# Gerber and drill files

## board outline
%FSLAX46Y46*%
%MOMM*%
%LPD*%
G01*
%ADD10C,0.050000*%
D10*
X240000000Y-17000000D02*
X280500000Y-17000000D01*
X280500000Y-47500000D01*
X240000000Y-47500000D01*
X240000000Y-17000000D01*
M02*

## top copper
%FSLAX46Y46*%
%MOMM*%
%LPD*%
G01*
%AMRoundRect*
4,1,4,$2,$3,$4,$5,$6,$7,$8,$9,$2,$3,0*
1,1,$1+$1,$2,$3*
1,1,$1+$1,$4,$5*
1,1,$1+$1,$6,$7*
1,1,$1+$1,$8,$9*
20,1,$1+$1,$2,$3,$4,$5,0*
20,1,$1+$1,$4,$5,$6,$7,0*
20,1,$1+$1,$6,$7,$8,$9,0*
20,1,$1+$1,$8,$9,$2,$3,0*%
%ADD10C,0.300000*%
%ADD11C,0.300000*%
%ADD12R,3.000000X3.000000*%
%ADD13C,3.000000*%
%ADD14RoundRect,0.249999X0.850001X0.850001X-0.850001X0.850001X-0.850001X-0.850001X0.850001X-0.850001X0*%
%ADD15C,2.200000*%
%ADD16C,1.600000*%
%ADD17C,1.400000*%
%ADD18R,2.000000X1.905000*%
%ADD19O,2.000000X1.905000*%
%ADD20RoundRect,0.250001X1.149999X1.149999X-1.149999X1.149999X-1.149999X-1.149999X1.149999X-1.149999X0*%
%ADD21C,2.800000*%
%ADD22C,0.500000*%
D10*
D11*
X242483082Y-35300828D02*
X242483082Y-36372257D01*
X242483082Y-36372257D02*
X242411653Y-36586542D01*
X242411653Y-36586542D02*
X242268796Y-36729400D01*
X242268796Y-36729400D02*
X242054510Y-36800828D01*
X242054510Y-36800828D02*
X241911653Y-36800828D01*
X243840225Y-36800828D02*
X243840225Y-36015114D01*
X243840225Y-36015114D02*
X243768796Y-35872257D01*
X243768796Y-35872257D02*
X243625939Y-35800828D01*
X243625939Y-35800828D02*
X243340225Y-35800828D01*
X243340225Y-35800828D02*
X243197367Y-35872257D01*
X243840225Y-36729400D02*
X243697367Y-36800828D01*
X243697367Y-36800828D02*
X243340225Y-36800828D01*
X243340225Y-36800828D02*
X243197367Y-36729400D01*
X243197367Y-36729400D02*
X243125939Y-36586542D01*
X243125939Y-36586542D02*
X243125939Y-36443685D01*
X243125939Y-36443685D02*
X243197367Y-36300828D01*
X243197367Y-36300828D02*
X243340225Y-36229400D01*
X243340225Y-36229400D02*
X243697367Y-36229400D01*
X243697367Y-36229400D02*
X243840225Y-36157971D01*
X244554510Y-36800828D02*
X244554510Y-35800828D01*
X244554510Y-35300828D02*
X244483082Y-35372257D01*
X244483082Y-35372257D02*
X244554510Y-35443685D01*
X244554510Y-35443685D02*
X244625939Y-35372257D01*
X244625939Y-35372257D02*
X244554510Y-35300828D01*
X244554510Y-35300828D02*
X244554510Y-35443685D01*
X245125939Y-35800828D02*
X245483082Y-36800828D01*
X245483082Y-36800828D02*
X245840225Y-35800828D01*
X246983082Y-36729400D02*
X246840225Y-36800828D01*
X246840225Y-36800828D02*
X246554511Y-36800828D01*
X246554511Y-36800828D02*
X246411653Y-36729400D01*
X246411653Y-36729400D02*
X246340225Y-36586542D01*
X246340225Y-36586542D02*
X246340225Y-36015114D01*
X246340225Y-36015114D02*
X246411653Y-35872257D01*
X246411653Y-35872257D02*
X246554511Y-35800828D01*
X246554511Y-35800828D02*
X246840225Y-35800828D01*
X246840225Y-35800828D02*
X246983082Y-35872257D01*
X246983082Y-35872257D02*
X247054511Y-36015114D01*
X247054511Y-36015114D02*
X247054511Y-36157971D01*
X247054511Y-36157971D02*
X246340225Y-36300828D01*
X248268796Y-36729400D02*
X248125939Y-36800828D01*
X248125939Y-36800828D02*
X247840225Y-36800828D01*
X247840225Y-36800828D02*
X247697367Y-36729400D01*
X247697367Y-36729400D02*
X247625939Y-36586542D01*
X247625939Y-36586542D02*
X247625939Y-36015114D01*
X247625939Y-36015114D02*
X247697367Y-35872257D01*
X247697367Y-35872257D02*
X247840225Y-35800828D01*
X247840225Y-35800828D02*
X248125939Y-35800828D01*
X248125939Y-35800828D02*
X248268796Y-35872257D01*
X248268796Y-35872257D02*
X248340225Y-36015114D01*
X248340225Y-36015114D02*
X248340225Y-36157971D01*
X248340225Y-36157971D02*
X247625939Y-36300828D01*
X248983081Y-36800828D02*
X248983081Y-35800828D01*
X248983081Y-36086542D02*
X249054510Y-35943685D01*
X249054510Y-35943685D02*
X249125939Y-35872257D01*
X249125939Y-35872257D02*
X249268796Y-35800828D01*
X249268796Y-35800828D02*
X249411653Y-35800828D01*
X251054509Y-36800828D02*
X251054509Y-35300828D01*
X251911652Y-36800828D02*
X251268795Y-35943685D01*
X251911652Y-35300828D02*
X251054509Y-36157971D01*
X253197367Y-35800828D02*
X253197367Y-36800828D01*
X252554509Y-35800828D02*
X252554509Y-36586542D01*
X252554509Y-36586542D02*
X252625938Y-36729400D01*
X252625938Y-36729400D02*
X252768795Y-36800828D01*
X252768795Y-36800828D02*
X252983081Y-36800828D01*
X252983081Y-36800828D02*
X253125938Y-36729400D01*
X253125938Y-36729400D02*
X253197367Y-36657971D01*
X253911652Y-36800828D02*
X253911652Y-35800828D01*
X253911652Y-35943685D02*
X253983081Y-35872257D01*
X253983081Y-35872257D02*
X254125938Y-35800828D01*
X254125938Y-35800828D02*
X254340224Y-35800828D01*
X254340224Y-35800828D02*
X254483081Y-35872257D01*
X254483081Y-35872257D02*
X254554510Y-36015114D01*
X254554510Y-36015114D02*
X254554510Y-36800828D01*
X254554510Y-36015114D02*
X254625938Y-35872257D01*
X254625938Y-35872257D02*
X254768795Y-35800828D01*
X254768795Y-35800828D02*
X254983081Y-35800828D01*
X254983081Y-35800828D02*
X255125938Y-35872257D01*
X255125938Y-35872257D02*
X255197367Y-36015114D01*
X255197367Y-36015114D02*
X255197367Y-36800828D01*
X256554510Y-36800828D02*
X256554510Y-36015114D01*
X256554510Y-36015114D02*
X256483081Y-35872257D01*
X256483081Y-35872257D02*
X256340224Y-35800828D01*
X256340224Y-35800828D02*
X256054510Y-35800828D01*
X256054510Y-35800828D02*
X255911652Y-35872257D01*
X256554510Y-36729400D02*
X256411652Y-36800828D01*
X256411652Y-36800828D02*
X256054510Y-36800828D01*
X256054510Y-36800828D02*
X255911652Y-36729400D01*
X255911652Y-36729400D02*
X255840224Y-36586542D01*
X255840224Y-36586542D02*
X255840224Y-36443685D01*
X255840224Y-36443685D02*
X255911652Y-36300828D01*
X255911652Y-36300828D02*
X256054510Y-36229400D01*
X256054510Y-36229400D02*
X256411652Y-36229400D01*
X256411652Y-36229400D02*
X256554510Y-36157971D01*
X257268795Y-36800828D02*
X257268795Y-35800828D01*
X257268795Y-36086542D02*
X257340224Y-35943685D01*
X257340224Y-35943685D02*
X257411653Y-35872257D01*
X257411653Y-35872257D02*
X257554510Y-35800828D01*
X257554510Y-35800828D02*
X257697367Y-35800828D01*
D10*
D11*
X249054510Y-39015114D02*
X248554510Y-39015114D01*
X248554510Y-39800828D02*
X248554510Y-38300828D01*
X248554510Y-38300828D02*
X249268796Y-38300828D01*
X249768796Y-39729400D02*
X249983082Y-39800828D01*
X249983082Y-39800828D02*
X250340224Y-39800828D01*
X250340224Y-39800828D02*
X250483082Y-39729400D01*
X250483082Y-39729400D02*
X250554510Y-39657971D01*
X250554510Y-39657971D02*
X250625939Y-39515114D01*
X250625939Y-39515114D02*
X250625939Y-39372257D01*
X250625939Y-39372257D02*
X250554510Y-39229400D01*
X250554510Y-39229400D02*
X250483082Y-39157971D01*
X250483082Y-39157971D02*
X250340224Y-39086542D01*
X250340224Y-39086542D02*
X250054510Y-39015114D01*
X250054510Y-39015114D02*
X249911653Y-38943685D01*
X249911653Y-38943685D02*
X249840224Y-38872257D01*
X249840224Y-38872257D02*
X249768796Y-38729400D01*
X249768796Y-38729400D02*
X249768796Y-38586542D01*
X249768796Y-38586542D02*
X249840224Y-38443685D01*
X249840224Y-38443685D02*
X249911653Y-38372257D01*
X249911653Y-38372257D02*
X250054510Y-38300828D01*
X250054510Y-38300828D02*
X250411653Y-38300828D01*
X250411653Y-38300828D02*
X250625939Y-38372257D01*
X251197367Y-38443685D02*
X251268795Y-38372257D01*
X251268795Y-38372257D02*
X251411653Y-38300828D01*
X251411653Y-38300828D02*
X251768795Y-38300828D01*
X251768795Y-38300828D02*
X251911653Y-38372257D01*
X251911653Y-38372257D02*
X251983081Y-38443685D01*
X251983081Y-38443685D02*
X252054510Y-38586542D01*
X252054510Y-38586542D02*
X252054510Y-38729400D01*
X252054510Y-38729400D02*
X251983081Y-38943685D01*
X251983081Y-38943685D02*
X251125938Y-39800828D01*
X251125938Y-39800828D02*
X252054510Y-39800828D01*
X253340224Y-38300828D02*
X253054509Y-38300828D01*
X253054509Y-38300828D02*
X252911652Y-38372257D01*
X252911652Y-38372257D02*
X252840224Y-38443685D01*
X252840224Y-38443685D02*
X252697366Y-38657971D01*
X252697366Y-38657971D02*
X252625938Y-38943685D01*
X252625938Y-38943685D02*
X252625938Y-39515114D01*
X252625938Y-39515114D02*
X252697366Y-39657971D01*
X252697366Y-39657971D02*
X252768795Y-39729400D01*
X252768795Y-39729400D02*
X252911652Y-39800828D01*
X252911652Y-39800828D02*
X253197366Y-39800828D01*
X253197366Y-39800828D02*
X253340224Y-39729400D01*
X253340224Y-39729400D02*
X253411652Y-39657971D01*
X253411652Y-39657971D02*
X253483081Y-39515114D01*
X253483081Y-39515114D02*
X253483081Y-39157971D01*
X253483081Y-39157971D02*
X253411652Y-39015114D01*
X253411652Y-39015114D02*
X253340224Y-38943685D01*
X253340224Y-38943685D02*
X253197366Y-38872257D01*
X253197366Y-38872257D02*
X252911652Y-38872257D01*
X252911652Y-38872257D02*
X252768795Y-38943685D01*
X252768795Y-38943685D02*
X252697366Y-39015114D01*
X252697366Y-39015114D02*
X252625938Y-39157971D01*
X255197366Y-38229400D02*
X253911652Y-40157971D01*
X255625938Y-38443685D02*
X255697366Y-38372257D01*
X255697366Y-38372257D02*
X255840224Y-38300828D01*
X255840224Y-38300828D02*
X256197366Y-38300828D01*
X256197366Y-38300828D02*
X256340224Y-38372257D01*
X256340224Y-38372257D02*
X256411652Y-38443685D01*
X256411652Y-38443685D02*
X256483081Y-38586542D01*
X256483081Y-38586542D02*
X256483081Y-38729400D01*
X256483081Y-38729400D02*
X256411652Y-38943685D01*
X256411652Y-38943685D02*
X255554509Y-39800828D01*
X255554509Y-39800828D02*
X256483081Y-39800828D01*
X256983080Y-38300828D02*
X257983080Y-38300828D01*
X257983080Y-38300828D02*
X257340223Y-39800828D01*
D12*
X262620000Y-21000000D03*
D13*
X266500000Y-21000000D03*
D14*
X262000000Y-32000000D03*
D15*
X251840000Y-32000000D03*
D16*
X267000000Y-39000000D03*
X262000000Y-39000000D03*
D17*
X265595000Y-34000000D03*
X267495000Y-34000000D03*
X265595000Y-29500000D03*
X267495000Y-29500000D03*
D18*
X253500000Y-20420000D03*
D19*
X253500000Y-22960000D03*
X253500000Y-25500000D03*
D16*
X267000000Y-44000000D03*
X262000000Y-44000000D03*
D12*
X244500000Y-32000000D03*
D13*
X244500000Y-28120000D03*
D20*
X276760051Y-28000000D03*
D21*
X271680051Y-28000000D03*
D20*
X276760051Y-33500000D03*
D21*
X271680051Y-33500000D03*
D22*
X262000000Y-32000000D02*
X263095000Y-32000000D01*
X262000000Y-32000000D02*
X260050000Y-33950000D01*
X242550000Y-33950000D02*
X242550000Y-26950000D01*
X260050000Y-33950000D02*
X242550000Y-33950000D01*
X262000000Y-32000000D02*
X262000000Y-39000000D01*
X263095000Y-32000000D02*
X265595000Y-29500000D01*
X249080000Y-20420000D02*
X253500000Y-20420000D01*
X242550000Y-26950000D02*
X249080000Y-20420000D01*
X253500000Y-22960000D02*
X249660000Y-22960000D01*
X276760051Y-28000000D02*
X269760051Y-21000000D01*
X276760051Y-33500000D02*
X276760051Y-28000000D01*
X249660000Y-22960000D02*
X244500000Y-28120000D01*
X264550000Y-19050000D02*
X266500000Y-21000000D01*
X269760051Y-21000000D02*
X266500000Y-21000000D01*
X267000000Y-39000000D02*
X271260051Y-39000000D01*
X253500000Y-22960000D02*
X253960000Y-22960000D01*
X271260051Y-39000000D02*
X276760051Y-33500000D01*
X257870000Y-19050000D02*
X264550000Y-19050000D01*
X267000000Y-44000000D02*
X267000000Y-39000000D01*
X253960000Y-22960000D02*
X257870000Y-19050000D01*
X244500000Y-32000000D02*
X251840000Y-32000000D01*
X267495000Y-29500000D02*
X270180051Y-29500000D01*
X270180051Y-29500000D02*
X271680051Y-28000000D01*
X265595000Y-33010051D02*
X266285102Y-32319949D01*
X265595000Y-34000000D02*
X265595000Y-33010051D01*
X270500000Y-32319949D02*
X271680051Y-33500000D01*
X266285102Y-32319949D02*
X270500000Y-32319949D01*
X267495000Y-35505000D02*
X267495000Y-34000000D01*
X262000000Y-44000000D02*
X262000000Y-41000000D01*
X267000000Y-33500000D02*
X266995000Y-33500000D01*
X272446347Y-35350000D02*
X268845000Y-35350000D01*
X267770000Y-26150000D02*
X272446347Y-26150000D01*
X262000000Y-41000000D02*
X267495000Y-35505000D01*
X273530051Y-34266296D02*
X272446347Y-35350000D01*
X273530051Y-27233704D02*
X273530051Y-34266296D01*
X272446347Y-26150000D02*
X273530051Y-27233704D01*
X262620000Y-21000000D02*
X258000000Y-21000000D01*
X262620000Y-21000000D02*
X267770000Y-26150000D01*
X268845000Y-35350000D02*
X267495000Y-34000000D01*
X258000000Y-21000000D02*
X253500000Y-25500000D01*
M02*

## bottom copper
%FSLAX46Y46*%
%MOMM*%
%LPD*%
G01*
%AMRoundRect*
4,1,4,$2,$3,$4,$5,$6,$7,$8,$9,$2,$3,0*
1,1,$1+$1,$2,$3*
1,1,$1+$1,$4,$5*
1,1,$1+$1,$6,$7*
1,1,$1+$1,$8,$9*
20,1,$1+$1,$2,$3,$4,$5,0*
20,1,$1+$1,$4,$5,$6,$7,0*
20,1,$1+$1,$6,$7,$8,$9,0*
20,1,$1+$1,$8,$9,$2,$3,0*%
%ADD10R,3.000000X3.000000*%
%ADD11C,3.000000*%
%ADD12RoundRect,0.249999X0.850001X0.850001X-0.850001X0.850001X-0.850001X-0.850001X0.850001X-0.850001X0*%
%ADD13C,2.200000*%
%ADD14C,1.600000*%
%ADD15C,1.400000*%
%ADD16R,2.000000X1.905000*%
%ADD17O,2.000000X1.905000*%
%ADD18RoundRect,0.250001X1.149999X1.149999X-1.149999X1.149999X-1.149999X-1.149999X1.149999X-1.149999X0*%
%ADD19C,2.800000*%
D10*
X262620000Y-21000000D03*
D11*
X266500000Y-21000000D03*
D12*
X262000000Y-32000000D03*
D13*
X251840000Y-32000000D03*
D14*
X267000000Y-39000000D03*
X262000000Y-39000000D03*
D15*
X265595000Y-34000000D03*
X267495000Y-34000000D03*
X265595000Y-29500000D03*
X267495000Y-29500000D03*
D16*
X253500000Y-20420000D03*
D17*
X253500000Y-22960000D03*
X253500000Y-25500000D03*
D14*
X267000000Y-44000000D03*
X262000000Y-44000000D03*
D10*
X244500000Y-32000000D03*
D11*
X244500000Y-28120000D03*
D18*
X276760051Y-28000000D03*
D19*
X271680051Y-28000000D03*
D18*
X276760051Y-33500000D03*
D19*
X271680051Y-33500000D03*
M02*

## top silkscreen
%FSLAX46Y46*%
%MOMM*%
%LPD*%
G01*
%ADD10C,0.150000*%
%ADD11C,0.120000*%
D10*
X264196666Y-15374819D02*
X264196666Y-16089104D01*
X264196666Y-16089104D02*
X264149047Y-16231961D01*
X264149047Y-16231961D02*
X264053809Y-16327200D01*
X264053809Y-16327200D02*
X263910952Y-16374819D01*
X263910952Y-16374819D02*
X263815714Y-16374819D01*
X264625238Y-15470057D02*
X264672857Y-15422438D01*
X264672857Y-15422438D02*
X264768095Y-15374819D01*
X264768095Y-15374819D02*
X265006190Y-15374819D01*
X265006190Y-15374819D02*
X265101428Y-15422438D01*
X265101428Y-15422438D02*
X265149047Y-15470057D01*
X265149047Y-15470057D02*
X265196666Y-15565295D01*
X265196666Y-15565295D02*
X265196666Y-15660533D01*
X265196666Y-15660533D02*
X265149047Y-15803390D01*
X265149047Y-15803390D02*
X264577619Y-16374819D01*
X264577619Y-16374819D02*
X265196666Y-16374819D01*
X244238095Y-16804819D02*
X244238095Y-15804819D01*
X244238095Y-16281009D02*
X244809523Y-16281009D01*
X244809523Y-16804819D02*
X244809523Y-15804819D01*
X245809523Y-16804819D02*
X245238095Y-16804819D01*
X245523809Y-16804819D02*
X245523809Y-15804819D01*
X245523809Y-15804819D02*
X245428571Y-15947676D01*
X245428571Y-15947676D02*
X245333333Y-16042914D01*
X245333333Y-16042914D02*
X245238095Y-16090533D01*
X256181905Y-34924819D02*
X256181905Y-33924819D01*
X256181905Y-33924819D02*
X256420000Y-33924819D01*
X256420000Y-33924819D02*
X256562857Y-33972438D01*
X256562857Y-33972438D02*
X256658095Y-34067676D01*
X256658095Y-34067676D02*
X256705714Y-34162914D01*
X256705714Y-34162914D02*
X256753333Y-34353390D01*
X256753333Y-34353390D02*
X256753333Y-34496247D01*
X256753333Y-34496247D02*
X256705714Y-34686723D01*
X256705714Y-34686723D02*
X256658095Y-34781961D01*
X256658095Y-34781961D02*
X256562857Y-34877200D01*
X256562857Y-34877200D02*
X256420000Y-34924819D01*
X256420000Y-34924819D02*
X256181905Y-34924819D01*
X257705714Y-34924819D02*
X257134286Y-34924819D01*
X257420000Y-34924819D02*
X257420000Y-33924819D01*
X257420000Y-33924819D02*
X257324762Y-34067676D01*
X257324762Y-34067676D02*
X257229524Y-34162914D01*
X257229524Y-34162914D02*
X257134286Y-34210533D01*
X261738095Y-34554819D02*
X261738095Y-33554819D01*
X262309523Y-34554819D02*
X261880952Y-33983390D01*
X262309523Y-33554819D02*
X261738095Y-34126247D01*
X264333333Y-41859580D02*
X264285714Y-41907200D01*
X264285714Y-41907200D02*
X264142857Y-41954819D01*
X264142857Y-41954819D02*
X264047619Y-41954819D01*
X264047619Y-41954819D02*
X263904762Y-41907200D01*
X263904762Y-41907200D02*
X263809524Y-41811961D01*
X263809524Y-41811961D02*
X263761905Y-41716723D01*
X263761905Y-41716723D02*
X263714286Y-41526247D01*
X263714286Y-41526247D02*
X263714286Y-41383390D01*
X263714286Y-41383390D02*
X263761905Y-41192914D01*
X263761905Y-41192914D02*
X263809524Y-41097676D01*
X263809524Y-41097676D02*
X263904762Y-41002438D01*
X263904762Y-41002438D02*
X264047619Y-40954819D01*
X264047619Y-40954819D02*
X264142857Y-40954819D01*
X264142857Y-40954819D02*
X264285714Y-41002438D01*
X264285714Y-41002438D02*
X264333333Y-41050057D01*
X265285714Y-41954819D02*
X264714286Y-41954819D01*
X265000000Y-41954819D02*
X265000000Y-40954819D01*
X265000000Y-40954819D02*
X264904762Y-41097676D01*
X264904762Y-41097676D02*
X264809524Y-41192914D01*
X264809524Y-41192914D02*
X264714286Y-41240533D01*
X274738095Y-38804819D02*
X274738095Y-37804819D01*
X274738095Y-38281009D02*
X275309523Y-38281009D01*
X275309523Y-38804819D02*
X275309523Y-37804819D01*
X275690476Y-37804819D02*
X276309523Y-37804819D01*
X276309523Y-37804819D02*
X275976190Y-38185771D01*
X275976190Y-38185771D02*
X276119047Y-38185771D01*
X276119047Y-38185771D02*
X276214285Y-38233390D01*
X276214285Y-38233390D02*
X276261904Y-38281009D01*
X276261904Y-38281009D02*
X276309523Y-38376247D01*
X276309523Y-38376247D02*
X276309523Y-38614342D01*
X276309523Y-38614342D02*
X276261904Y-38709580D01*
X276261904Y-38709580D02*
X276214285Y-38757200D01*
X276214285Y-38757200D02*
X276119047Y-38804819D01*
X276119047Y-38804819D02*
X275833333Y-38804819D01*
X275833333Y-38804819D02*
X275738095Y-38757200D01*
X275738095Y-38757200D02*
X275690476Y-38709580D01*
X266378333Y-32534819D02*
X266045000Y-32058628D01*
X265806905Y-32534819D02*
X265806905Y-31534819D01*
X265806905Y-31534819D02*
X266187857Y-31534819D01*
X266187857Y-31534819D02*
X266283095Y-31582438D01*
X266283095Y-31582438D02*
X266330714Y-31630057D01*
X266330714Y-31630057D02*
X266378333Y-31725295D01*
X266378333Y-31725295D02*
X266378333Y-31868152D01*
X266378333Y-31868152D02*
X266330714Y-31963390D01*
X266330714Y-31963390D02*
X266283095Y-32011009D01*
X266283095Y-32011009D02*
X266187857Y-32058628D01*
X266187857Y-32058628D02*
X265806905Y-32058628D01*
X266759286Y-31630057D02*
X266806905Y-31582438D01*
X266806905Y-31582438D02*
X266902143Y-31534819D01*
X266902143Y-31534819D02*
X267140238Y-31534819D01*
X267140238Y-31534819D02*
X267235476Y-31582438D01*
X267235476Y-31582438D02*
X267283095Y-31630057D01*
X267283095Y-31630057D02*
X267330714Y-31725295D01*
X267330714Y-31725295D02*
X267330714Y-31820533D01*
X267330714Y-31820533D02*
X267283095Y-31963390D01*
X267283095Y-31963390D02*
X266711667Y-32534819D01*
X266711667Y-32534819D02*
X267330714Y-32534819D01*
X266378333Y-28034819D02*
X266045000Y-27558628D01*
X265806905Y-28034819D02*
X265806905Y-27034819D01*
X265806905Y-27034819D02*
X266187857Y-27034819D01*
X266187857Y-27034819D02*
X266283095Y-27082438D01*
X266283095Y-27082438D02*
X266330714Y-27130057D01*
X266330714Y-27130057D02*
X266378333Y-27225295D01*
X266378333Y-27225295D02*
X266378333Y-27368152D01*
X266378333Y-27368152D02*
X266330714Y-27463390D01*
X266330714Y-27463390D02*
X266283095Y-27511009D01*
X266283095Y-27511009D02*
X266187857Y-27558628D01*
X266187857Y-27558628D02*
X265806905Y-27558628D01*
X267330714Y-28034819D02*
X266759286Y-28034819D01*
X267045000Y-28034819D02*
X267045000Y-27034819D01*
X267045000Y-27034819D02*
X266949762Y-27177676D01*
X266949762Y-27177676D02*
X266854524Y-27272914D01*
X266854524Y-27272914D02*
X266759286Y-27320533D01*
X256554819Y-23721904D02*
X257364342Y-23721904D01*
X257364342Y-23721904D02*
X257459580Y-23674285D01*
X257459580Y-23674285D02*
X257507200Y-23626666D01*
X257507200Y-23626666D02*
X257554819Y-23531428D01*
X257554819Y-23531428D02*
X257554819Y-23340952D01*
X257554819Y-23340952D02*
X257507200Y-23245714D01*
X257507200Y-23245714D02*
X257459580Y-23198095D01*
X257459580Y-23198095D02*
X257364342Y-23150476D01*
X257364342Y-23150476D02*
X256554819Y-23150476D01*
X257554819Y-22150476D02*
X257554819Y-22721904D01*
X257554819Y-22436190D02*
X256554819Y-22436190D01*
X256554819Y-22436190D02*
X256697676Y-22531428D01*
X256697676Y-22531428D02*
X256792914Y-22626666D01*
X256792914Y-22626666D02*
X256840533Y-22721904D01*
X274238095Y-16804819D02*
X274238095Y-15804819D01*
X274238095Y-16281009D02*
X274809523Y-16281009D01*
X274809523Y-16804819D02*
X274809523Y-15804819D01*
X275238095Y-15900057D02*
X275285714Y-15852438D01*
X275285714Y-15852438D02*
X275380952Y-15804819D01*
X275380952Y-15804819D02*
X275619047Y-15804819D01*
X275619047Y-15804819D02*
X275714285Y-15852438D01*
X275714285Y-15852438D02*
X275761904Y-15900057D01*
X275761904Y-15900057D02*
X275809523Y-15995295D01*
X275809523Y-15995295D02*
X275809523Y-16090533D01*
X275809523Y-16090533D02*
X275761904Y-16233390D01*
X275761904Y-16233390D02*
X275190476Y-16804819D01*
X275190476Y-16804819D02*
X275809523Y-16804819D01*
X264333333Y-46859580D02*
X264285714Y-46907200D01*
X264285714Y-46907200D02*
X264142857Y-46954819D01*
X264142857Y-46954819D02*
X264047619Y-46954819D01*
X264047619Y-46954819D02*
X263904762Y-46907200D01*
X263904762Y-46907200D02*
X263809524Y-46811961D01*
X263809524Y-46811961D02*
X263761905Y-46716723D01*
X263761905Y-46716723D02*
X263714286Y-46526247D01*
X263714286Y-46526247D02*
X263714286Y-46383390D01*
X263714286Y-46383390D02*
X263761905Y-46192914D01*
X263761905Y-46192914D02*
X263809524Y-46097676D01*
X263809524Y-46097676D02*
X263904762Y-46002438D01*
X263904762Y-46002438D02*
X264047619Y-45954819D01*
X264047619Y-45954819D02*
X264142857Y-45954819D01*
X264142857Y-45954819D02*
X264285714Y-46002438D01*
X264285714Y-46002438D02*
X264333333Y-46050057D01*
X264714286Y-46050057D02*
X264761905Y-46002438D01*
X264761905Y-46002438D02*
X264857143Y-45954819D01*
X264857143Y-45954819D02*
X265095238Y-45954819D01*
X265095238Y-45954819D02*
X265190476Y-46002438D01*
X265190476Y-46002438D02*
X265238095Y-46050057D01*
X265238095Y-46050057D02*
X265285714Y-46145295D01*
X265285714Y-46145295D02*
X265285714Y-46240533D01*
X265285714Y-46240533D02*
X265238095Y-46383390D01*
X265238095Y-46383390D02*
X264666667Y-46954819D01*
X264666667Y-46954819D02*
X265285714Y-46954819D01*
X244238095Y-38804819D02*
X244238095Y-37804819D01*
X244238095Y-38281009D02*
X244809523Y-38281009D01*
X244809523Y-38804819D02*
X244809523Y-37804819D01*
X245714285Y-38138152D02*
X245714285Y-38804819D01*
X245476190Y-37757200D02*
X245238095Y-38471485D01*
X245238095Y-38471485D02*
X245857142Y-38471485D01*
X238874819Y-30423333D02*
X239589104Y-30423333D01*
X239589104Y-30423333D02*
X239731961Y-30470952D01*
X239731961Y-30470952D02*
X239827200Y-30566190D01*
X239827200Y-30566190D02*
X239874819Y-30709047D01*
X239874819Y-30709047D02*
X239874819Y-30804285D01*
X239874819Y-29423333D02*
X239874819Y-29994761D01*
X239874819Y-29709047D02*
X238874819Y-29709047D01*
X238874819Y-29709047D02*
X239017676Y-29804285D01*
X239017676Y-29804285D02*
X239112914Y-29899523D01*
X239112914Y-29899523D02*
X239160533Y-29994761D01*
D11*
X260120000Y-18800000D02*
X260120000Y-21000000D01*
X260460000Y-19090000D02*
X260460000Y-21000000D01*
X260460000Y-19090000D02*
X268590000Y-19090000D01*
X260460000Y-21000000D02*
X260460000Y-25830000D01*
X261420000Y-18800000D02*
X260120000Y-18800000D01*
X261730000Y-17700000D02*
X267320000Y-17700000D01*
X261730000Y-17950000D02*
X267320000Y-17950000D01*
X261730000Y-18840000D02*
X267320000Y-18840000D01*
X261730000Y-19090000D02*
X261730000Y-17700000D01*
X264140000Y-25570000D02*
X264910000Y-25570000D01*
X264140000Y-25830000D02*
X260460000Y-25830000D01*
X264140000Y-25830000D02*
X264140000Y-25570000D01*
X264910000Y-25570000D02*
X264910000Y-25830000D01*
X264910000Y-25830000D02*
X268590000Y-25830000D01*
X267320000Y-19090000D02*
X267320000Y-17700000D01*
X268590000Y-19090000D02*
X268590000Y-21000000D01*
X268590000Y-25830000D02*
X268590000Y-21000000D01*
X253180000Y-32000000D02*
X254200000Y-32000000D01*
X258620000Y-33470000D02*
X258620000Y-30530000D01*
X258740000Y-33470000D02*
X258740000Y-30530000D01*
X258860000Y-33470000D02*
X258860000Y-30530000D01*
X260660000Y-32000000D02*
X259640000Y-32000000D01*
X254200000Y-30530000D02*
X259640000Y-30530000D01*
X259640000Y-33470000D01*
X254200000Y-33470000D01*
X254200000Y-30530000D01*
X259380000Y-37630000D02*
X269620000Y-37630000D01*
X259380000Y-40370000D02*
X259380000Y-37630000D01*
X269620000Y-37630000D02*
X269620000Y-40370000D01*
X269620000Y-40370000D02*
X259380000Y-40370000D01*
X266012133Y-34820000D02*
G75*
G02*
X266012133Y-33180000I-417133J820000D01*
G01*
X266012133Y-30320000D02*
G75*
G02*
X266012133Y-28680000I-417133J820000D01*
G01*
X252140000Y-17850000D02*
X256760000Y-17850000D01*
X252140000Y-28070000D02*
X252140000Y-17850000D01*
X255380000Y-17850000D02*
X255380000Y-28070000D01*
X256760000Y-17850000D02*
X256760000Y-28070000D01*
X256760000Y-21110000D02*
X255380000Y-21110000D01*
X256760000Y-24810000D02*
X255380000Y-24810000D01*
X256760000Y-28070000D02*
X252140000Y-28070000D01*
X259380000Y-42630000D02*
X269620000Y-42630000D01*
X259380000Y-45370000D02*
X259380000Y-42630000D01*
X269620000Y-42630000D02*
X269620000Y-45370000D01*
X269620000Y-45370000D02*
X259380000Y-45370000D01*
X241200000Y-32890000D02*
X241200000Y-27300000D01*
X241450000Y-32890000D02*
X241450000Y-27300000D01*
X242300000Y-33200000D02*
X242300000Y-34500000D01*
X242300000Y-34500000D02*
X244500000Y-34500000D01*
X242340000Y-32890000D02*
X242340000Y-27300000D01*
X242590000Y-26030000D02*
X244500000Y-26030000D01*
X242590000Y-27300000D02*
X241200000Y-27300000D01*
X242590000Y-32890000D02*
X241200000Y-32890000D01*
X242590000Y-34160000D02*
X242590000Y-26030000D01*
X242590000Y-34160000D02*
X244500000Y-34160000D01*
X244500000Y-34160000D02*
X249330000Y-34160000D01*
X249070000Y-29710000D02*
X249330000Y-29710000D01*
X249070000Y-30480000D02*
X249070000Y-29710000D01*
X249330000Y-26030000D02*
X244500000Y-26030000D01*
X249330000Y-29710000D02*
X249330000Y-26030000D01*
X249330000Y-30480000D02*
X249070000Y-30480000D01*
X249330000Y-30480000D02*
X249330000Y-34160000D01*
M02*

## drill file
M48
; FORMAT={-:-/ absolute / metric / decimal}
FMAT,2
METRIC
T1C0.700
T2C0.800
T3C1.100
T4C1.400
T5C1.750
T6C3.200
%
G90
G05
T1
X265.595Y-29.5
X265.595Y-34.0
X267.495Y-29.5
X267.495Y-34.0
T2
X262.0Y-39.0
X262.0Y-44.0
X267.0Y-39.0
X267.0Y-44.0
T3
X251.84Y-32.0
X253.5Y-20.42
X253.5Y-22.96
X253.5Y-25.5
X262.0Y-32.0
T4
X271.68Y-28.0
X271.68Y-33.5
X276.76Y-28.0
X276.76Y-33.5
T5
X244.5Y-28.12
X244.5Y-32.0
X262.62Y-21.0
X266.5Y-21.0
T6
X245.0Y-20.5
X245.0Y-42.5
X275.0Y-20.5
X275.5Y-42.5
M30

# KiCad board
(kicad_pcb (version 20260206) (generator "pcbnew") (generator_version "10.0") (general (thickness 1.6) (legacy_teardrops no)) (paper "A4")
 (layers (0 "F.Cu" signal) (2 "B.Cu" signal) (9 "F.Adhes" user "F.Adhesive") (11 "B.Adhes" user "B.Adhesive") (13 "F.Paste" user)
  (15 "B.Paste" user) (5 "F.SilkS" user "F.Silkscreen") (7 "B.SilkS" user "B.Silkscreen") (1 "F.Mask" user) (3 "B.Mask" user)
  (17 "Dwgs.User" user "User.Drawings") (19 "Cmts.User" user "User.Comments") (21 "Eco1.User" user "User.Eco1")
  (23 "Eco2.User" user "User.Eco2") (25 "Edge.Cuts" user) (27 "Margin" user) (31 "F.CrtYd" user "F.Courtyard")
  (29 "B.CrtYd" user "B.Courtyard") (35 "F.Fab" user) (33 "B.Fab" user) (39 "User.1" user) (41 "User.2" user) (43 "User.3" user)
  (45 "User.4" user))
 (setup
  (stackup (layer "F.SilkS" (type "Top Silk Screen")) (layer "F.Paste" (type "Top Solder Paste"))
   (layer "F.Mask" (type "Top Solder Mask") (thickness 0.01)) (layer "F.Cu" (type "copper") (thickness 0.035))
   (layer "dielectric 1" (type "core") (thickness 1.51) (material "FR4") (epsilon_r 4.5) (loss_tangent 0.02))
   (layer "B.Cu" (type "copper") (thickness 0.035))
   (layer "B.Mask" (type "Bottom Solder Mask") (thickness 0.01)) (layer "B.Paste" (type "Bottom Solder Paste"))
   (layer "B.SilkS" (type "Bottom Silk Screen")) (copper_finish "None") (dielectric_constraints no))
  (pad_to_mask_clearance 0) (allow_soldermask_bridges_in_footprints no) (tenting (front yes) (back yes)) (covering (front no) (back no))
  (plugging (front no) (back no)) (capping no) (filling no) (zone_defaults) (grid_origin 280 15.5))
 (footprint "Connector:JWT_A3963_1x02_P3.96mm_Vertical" (layer "F.Cu") (at 262.62 21)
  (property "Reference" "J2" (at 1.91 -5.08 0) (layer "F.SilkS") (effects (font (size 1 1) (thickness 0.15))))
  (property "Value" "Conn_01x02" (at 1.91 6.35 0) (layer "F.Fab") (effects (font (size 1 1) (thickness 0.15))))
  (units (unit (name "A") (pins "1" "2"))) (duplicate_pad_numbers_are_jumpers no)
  (fp_line (start -2.5 -2.2) (end -2.5 0) (stroke (width 0.12) (type solid)) (layer "F.SilkS"))
  (fp_line (start -2.16 -1.91) (end -2.16 0) (stroke (width 0.12) (type solid)) (layer "F.SilkS"))
  (fp_line (start -2.16 -1.91) (end 5.97 -1.91) (stroke (width 0.12) (type solid)) (layer "F.SilkS"))
  (fp_line (start -2.16 0) (end -2.16 4.83) (stroke (width 0.12) (type solid)) (layer "F.SilkS"))
  (fp_line (start -1.2 -2.2) (end -2.5 -2.2) (stroke (width 0.12) (type solid)) (layer "F.SilkS"))
  (fp_line (start -0.89 -3.3) (end 4.7 -3.3) (stroke (width 0.12) (type solid)) (layer "F.SilkS"))
  (fp_line (start -0.89 -3.05) (end 4.7 -3.05) (stroke (width 0.12) (type solid)) (layer "F.SilkS"))
  (fp_line (start -0.89 -2.16) (end 4.7 -2.16) (stroke (width 0.12) (type solid)) (layer "F.SilkS"))
  (fp_line (start -0.89 -1.91) (end -0.89 -3.3) (stroke (width 0.12) (type solid)) (layer "F.SilkS"))
  (fp_line (start 1.52 4.57) (end 2.29 4.57) (stroke (width 0.12) (type solid)) (layer "F.SilkS"))
  (fp_line (start 1.52 4.83) (end -2.16 4.83) (stroke (width 0.12) (type solid)) (layer "F.SilkS"))
  (fp_line (start 1.52 4.83) (end 1.52 4.57) (stroke (width 0.12) (type solid)) (layer "F.SilkS"))
  (fp_line (start 2.29 4.57) (end 2.29 4.83) (stroke (width 0.12) (type solid)) (layer "F.SilkS"))
  (fp_line (start 2.29 4.83) (end 5.97 4.83) (stroke (width 0.12) (type solid)) (layer "F.SilkS"))
  (fp_line (start 4.7 -1.91) (end 4.7 -3.3) (stroke (width 0.12) (type solid)) (layer "F.SilkS"))
  (fp_line (start 5.97 -1.91) (end 5.97 0) (stroke (width 0.12) (type solid)) (layer "F.SilkS"))
  (fp_line (start 5.97 4.83) (end 5.97 0) (stroke (width 0.12) (type solid)) (layer "F.SilkS"))
  (pad "1" thru_hole rect (at 0 0) (size 3 3) (drill 1.75) (layers "*.Cu" "*.Mask") (remove_unused_layers no) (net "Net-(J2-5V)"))
  (pad "2" thru_hole circle (at 3.88 0) (size 3 3) (drill 1.75) (layers "*.Cu" "*.Mask") (remove_unused_layers no) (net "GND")))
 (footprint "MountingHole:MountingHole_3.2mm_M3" (layer "F.Cu") (at 245 20.5)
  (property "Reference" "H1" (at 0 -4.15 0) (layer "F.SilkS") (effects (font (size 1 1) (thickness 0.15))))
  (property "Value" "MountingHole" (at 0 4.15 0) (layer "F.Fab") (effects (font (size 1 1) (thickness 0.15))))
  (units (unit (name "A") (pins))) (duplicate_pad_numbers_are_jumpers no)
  (pad "" np_thru_hole circle (at 0 0) (size 3.2 3.2) (drill 3.2) (layers "*.Cu" "*.Mask")))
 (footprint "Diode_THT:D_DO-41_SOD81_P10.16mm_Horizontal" (layer "F.Cu") (at 262 32 180)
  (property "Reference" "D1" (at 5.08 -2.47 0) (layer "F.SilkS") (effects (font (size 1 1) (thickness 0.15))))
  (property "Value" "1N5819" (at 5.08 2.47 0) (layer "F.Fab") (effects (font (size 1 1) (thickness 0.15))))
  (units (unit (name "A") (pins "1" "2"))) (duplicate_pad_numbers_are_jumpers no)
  (fp_line (start 8.82 0) (end 7.8 0) (stroke (width 0.12) (type solid)) (layer "F.SilkS"))
  (fp_line (start 3.38 -1.47) (end 3.38 1.47) (stroke (width 0.12) (type solid)) (layer "F.SilkS"))
  (fp_line (start 3.26 -1.47) (end 3.26 1.47) (stroke (width 0.12) (type solid)) (layer "F.SilkS"))
  (fp_line (start 3.14 -1.47) (end 3.14 1.47) (stroke (width 0.12) (type solid)) (layer "F.SilkS"))
  (fp_line (start 1.34 0) (end 2.36 0) (stroke (width 0.12) (type solid)) (layer "F.SilkS"))
  (fp_rect (start 2.36 -1.47) (end 7.8 1.47) (stroke (width 0.12) (type solid)) (fill no) (layer "F.SilkS"))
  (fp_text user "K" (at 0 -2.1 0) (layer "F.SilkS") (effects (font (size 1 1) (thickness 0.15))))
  (pad "1" thru_hole roundrect (at 0 0 180) (size 2.2 2.2) (drill 1.1) (layers "*.Cu" "*.Mask") (remove_unused_layers no)
   (roundrect_rratio 0.113636) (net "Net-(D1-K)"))
  (pad "2" thru_hole circle (at 10.16 0 180) (size 2.2 2.2) (drill 1.1) (layers "*.Cu" "*.Mask") (remove_unused_layers no)
   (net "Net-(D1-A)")))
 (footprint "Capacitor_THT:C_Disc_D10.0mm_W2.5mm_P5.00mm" (layer "F.Cu") (at 267 39 180)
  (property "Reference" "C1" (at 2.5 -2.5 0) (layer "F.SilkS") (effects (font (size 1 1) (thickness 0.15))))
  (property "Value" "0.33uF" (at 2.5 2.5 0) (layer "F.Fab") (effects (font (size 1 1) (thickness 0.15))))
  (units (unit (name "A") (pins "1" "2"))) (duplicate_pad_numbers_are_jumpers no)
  (fp_line (start 7.62 1.37) (end -2.62 1.37) (stroke (width 0.12) (type solid)) (layer "F.SilkS"))
  (fp_line (start 7.62 -1.37) (end 7.62 1.37) (stroke (width 0.12) (type solid)) (layer "F.SilkS"))
  (fp_line (start -2.62 1.37) (end -2.62 -1.37) (stroke (width 0.12) (type solid)) (layer "F.SilkS"))
  (fp_line (start -2.62 -1.37) (end 7.62 -1.37) (stroke (width 0.12) (type solid)) (layer "F.SilkS"))
  (pad "1" thru_hole circle (at 0 0 180) (size 1.6 1.6) (drill 0.8) (layers "*.Cu" "*.Mask") (remove_unused_layers no) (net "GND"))
  (pad "2" thru_hole circle (at 5 0 180) (size 1.6 1.6) (drill 0.8) (layers "*.Cu" "*.Mask") (remove_unused_layers no) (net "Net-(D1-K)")))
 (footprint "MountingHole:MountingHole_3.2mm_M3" (layer "F.Cu") (at 275.5 42.5)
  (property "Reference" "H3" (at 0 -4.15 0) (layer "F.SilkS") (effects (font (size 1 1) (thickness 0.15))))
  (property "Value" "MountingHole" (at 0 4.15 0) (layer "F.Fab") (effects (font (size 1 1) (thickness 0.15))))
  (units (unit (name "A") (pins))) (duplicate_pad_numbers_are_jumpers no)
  (pad "" np_thru_hole circle (at 0 0) (size 3.2 3.2) (drill 3.2) (layers "*.Cu" "*.Mask")))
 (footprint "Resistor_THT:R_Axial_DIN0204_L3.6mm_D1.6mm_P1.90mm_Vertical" (layer "F.Cu") (at 265.595 34)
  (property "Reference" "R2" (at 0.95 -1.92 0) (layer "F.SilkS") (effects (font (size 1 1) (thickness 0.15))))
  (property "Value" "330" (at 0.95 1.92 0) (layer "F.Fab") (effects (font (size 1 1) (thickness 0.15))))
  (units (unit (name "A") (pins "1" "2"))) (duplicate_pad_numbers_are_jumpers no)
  (fp_arc (start 0.417133 0.82) (mid -0.92 0) (end 0.417133 -0.82) (stroke (width 0.12) (type solid)) (layer "F.SilkS"))
  (pad "1" thru_hole circle (at 0 0) (size 1.4 1.4) (drill 0.7) (layers "*.Cu" "*.Mask") (remove_unused_layers no) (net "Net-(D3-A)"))
  (pad "2" thru_hole circle (at 1.9 0) (size 1.4 1.4) (drill 0.7) (layers "*.Cu" "*.Mask") (remove_unused_layers no) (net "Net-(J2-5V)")))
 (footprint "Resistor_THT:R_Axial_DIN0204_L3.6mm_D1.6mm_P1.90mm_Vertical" (layer "F.Cu") (at 265.595 29.5)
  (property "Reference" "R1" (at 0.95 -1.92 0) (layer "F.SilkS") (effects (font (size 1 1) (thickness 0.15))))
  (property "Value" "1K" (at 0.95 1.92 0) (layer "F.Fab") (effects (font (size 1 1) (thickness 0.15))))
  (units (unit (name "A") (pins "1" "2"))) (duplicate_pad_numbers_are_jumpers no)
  (fp_arc (start 0.417133 0.82) (mid -0.92 0) (end 0.417133 -0.82) (stroke (width 0.12) (type solid)) (layer "F.SilkS"))
  (pad "1" thru_hole circle (at 0 0) (size 1.4 1.4) (drill 0.7) (layers "*.Cu" "*.Mask") (remove_unused_layers no) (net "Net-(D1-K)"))
  (pad "2" thru_hole circle (at 1.9 0) (size 1.4 1.4) (drill 0.7) (layers "*.Cu" "*.Mask") (remove_unused_layers no) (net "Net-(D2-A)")))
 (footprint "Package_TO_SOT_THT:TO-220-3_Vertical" (layer "F.Cu") (at 253.5 20.42 -90)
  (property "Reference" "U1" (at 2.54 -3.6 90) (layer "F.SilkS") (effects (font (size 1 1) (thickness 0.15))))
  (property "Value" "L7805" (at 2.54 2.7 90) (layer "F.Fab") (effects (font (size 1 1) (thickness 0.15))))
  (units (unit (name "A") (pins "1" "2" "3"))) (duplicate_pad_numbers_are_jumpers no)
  (fp_line (start -2.57 1.36) (end -2.57 -3.26) (stroke (width 0.12) (type solid)) (layer "F.SilkS"))
  (fp_line (start 7.65 1.36) (end -2.57 1.36) (stroke (width 0.12) (type solid)) (layer "F.SilkS"))
  (fp_line (start -2.57 -1.88) (end 7.65 -1.88) (stroke (width 0.12) (type solid)) (layer "F.SilkS"))
  (fp_line (start -2.57 -3.26) (end 7.65 -3.26) (stroke (width 0.12) (type solid)) (layer "F.SilkS"))
  (fp_line (start 0.69 -3.26) (end 0.69 -1.88) (stroke (width 0.12) (type solid)) (layer "F.SilkS"))
  (fp_line (start 4.39 -3.26) (end 4.39 -1.88) (stroke (width 0.12) (type solid)) (layer "F.SilkS"))
  (fp_line (start 7.65 -3.26) (end 7.65 1.36) (stroke (width 0.12) (type solid)) (layer "F.SilkS"))
  (pad "1" thru_hole rect (at 0 0 270) (size 1.905 2) (drill 1.1) (layers "*.Cu" "*.Mask") (remove_unused_layers no) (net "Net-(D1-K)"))
  (pad "2" thru_hole oval (at 2.54 0 270) (size 1.905 2) (drill 1.1) (layers "*.Cu" "*.Mask") (remove_unused_layers no) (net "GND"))
  (pad "3" thru_hole oval (at 5.08 0 270) (size 1.905 2) (drill 1.1) (layers "*.Cu" "*.Mask") (remove_unused_layers no) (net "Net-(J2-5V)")))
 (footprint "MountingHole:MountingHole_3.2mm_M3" (layer "F.Cu") (at 275 20.5)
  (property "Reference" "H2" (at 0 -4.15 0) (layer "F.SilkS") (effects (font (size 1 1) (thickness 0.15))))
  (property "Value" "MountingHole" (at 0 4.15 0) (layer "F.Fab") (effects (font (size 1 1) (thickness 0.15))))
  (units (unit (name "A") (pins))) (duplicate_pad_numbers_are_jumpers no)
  (pad "" np_thru_hole circle (at 0 0) (size 3.2 3.2) (drill 3.2) (layers "*.Cu" "*.Mask")))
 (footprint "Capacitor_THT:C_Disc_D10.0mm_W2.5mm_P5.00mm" (layer "F.Cu") (at 267 44 180)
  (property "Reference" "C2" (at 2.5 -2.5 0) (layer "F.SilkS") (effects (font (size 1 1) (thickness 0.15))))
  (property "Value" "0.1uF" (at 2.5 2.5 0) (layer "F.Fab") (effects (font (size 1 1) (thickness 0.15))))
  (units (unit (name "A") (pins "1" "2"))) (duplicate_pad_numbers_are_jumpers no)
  (fp_line (start 7.62 1.37) (end -2.62 1.37) (stroke (width 0.12) (type solid)) (layer "F.SilkS"))
  (fp_line (start 7.62 -1.37) (end 7.62 1.37) (stroke (width 0.12) (type solid)) (layer "F.SilkS"))
  (fp_line (start -2.62 1.37) (end -2.62 -1.37) (stroke (width 0.12) (type solid)) (layer "F.SilkS"))
  (fp_line (start -2.62 -1.37) (end 7.62 -1.37) (stroke (width 0.12) (type solid)) (layer "F.SilkS"))
  (pad "1" thru_hole circle (at 0 0 180) (size 1.6 1.6) (drill 0.8) (layers "*.Cu" "*.Mask") (remove_unused_layers no) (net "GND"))
  (pad "2" thru_hole circle (at 5 0 180) (size 1.6 1.6) (drill 0.8) (layers "*.Cu" "*.Mask") (remove_unused_layers no) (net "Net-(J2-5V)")))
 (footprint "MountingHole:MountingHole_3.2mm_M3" (layer "F.Cu") (at 245 42.5)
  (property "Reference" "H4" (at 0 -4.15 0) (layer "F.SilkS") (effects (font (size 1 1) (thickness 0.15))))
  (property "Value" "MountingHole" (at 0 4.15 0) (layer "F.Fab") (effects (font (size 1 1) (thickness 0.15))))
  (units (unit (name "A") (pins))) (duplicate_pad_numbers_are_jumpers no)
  (pad "" np_thru_hole circle (at 0 0) (size 3.2 3.2) (drill 3.2) (layers "*.Cu" "*.Mask")))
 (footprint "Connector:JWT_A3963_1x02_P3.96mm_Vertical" (layer "F.Cu") (at 244.5 32 90)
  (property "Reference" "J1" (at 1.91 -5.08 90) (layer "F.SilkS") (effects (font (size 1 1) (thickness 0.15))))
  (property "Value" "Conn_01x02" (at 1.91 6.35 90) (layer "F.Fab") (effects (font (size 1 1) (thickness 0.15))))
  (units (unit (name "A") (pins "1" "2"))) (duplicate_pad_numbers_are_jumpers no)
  (fp_line (start -0.89 -3.3) (end 4.7 -3.3) (stroke (width 0.12) (type solid)) (layer "F.SilkS"))
  (fp_line (start -0.89 -3.05) (end 4.7 -3.05) (stroke (width 0.12) (type solid)) (layer "F.SilkS"))
  (fp_line (start -1.2 -2.2) (end -2.5 -2.2) (stroke (width 0.12) (type solid)) (layer "F.SilkS"))
  (fp_line (start -2.5 -2.2) (end -2.5 0) (stroke (width 0.12) (type solid)) (layer "F.SilkS"))
  (fp_line (start -0.89 -2.16) (end 4.7 -2.16) (stroke (width 0.12) (type solid)) (layer "F.SilkS"))
  (fp_line (start 5.97 -1.91) (end 5.97 0) (stroke (width 0.12) (type solid)) (layer "F.SilkS"))
  (fp_line (start 4.7 -1.91) (end 4.7 -3.3) (stroke (width 0.12) (type solid)) (layer "F.SilkS"))
  (fp_line (start -0.89 -1.91) (end -0.89 -3.3) (stroke (width 0.12) (type solid)) (layer "F.SilkS"))
  (fp_line (start -2.16 -1.91) (end 5.97 -1.91) (stroke (width 0.12) (type solid)) (layer "F.SilkS"))
  (fp_line (start -2.16 -1.91) (end -2.16 0) (stroke (width 0.12) (type solid)) (layer "F.SilkS"))
  (fp_line (start -2.16 0) (end -2.16 4.83) (stroke (width 0.12) (type solid)) (layer "F.SilkS"))
  (fp_line (start 2.29 4.57) (end 2.29 4.83) (stroke (width 0.12) (type solid)) (layer "F.SilkS"))
  (fp_line (start 1.52 4.57) (end 2.29 4.57) (stroke (width 0.12) (type solid)) (layer "F.SilkS"))
  (fp_line (start 5.97 4.83) (end 5.97 0) (stroke (width 0.12) (type solid)) (layer "F.SilkS"))
  (fp_line (start 2.29 4.83) (end 5.97 4.83) (stroke (width 0.12) (type solid)) (layer "F.SilkS"))
  (fp_line (start 1.52 4.83) (end 1.52 4.57) (stroke (width 0.12) (type solid)) (layer "F.SilkS"))
  (fp_line (start 1.52 4.83) (end -2.16 4.83) (stroke (width 0.12) (type solid)) (layer "F.SilkS"))
  (pad "1" thru_hole rect (at 0 0 90) (size 3 3) (drill 1.75) (layers "*.Cu" "*.Mask") (remove_unused_layers no) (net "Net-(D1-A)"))
  (pad "2" thru_hole circle (at 3.88 0 90) (size 3 3) (drill 1.75) (layers "*.Cu" "*.Mask") (remove_unused_layers no) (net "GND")))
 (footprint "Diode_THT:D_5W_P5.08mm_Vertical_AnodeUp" (layer "B.Cu") (at 276.760051 28 180)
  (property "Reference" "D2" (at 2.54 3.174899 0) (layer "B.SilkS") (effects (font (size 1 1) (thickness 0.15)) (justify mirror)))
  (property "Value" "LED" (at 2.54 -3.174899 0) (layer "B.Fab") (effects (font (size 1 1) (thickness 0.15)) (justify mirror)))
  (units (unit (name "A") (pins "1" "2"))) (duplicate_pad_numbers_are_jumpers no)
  (pad "1" thru_hole roundrect (at 0 0 180) (size 2.8 2.8) (drill 1.4) (layers "*.Cu" "*.Mask") (remove_unused_layers no)
   (roundrect_rratio 0.089286) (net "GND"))
  (pad "2" thru_hole circle (at 5.08 0 180) (size 2.8 2.8) (drill 1.4) (layers "*.Cu" "*.Mask") (remove_unused_layers no) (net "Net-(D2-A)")))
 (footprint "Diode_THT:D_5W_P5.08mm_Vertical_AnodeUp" (layer "B.Cu") (at 276.760051 33.5 180)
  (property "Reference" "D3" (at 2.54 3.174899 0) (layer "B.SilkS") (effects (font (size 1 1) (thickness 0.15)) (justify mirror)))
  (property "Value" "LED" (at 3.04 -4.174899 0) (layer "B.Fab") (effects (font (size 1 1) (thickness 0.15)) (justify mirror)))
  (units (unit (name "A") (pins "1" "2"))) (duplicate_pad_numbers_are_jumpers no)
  (pad "1" thru_hole roundrect (at 0 0 180) (size 2.8 2.8) (drill 1.4) (layers "*.Cu" "*.Mask") (remove_unused_layers no)
   (roundrect_rratio 0.089286) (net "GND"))
  (pad "2" thru_hole circle (at 5.08 0 180) (size 2.8 2.8) (drill 1.4) (layers "*.Cu" "*.Mask") (remove_unused_layers no) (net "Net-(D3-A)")))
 (gr_rect (start 240 17) (end 280.5 47.5) (stroke (width 0.05) (type default)) (fill no) (layer "Edge.Cuts"))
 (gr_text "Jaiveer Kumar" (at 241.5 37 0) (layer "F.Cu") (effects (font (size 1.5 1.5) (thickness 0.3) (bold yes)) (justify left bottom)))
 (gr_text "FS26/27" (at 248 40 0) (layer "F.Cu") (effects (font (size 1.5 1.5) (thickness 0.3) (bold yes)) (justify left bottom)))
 (segment (start 262 32) (end 263.095 32) (width 0.5) (layer "F.Cu") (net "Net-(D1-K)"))
 (segment (start 262 32) (end 260.05 33.95) (width 0.5) (layer "F.Cu") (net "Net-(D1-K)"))
 (segment (start 242.55 33.95) (end 242.55 26.95) (width 0.5) (layer "F.Cu") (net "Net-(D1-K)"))
 (segment (start 260.05 33.95) (end 242.55 33.95) (width 0.5) (layer "F.Cu") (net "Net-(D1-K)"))
 (segment (start 262 32) (end 262 39) (width 0.5) (layer "F.Cu") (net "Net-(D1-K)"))
 (segment (start 263.095 32) (end 265.595 29.5) (width 0.5) (layer "F.Cu") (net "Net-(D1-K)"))
 (segment (start 249.08 20.42) (end 253.5 20.42) (width 0.5) (layer "F.Cu") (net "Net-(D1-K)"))
 (segment (start 242.55 26.95) (end 249.08 20.42) (width 0.5) (layer "F.Cu") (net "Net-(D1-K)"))
 (segment (start 253.5 22.96) (end 249.66 22.96) (width 0.5) (layer "F.Cu") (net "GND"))
 (segment (start 276.760051 28) (end 269.760051 21) (width 0.5) (layer "F.Cu") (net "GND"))
 (segment (start 276.760051 33.5) (end 276.760051 28) (width 0.5) (layer "F.Cu") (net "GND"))
 (segment (start 249.66 22.96) (end 244.5 28.12) (width 0.5) (layer "F.Cu") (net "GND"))
 (segment (start 264.55 19.05) (end 266.5 21) (width 0.5) (layer "F.Cu") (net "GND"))
 (segment (start 269.760051 21) (end 266.5 21) (width 0.5) (layer "F.Cu") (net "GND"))
 (segment (start 267 39) (end 271.260051 39) (width 0.5) (layer "F.Cu") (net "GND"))
 (segment (start 253.5 22.96) (end 253.96 22.96) (width 0.5) (layer "F.Cu") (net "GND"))
 (segment (start 271.260051 39) (end 276.760051 33.5) (width 0.5) (layer "F.Cu") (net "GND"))
 (segment (start 257.87 19.05) (end 264.55 19.05) (width 0.5) (layer "F.Cu") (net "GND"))
 (segment (start 267 44) (end 267 39) (width 0.5) (layer "F.Cu") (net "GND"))
 (segment (start 253.96 22.96) (end 257.87 19.05) (width 0.5) (layer "F.Cu") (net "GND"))
 (segment (start 244.5 32) (end 251.84 32) (width 0.5) (layer "F.Cu") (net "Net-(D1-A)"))
 (segment (start 267.495 29.5) (end 270.180051 29.5) (width 0.5) (layer "F.Cu") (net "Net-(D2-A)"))
 (segment (start 270.180051 29.5) (end 271.680051 28) (width 0.5) (layer "F.Cu") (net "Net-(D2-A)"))
 (segment (start 265.595 33.010051) (end 266.285102 32.319949) (width 0.5) (layer "F.Cu") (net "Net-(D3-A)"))
 (segment (start 265.595 34) (end 265.595 33.010051) (width 0.5) (layer "F.Cu") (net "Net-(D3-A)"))
 (segment (start 270.5 32.319949) (end 271.680051 33.5) (width 0.5) (layer "F.Cu") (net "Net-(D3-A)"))
 (segment (start 266.285102 32.319949) (end 270.5 32.319949) (width 0.5) (layer "F.Cu") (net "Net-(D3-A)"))
 (segment (start 267.495 35.505) (end 267.495 34) (width 0.5) (layer "F.Cu") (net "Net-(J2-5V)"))
 (segment (start 262 44) (end 262 41) (width 0.5) (layer "F.Cu") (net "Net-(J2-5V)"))
 (segment (start 267 33.5) (end 266.995 33.5) (width 0.5) (layer "F.Cu") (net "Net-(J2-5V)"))
 (segment (start 272.446347 35.35) (end 268.845 35.35) (width 0.5) (layer "F.Cu") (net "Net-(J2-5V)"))
 (segment (start 267.77 26.15) (end 272.446347 26.15) (width 0.5) (layer "F.Cu") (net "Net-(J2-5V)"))
 (segment (start 262 41) (end 267.495 35.505) (width 0.5) (layer "F.Cu") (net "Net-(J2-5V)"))
 (segment (start 273.530051 34.266296) (end 272.446347 35.35) (width 0.5) (layer "F.Cu") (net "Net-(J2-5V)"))
 (segment (start 273.530051 27.233704) (end 273.530051 34.266296) (width 0.5) (layer "F.Cu") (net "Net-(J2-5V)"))
 (segment (start 272.446347 26.15) (end 273.530051 27.233704) (width 0.5) (layer "F.Cu") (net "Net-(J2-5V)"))
 (segment (start 262.62 21) (end 258 21) (width 0.5) (layer "F.Cu") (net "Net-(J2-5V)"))
 (segment (start 262.62 21) (end 267.77 26.15) (width 0.5) (layer "F.Cu") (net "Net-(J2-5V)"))
 (segment (start 268.845 35.35) (end 267.495 34) (width 0.5) (layer "F.Cu") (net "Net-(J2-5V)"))
 (segment (start 258 21) (end 253.5 25.5) (width 0.5) (layer "F.Cu") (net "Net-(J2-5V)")))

